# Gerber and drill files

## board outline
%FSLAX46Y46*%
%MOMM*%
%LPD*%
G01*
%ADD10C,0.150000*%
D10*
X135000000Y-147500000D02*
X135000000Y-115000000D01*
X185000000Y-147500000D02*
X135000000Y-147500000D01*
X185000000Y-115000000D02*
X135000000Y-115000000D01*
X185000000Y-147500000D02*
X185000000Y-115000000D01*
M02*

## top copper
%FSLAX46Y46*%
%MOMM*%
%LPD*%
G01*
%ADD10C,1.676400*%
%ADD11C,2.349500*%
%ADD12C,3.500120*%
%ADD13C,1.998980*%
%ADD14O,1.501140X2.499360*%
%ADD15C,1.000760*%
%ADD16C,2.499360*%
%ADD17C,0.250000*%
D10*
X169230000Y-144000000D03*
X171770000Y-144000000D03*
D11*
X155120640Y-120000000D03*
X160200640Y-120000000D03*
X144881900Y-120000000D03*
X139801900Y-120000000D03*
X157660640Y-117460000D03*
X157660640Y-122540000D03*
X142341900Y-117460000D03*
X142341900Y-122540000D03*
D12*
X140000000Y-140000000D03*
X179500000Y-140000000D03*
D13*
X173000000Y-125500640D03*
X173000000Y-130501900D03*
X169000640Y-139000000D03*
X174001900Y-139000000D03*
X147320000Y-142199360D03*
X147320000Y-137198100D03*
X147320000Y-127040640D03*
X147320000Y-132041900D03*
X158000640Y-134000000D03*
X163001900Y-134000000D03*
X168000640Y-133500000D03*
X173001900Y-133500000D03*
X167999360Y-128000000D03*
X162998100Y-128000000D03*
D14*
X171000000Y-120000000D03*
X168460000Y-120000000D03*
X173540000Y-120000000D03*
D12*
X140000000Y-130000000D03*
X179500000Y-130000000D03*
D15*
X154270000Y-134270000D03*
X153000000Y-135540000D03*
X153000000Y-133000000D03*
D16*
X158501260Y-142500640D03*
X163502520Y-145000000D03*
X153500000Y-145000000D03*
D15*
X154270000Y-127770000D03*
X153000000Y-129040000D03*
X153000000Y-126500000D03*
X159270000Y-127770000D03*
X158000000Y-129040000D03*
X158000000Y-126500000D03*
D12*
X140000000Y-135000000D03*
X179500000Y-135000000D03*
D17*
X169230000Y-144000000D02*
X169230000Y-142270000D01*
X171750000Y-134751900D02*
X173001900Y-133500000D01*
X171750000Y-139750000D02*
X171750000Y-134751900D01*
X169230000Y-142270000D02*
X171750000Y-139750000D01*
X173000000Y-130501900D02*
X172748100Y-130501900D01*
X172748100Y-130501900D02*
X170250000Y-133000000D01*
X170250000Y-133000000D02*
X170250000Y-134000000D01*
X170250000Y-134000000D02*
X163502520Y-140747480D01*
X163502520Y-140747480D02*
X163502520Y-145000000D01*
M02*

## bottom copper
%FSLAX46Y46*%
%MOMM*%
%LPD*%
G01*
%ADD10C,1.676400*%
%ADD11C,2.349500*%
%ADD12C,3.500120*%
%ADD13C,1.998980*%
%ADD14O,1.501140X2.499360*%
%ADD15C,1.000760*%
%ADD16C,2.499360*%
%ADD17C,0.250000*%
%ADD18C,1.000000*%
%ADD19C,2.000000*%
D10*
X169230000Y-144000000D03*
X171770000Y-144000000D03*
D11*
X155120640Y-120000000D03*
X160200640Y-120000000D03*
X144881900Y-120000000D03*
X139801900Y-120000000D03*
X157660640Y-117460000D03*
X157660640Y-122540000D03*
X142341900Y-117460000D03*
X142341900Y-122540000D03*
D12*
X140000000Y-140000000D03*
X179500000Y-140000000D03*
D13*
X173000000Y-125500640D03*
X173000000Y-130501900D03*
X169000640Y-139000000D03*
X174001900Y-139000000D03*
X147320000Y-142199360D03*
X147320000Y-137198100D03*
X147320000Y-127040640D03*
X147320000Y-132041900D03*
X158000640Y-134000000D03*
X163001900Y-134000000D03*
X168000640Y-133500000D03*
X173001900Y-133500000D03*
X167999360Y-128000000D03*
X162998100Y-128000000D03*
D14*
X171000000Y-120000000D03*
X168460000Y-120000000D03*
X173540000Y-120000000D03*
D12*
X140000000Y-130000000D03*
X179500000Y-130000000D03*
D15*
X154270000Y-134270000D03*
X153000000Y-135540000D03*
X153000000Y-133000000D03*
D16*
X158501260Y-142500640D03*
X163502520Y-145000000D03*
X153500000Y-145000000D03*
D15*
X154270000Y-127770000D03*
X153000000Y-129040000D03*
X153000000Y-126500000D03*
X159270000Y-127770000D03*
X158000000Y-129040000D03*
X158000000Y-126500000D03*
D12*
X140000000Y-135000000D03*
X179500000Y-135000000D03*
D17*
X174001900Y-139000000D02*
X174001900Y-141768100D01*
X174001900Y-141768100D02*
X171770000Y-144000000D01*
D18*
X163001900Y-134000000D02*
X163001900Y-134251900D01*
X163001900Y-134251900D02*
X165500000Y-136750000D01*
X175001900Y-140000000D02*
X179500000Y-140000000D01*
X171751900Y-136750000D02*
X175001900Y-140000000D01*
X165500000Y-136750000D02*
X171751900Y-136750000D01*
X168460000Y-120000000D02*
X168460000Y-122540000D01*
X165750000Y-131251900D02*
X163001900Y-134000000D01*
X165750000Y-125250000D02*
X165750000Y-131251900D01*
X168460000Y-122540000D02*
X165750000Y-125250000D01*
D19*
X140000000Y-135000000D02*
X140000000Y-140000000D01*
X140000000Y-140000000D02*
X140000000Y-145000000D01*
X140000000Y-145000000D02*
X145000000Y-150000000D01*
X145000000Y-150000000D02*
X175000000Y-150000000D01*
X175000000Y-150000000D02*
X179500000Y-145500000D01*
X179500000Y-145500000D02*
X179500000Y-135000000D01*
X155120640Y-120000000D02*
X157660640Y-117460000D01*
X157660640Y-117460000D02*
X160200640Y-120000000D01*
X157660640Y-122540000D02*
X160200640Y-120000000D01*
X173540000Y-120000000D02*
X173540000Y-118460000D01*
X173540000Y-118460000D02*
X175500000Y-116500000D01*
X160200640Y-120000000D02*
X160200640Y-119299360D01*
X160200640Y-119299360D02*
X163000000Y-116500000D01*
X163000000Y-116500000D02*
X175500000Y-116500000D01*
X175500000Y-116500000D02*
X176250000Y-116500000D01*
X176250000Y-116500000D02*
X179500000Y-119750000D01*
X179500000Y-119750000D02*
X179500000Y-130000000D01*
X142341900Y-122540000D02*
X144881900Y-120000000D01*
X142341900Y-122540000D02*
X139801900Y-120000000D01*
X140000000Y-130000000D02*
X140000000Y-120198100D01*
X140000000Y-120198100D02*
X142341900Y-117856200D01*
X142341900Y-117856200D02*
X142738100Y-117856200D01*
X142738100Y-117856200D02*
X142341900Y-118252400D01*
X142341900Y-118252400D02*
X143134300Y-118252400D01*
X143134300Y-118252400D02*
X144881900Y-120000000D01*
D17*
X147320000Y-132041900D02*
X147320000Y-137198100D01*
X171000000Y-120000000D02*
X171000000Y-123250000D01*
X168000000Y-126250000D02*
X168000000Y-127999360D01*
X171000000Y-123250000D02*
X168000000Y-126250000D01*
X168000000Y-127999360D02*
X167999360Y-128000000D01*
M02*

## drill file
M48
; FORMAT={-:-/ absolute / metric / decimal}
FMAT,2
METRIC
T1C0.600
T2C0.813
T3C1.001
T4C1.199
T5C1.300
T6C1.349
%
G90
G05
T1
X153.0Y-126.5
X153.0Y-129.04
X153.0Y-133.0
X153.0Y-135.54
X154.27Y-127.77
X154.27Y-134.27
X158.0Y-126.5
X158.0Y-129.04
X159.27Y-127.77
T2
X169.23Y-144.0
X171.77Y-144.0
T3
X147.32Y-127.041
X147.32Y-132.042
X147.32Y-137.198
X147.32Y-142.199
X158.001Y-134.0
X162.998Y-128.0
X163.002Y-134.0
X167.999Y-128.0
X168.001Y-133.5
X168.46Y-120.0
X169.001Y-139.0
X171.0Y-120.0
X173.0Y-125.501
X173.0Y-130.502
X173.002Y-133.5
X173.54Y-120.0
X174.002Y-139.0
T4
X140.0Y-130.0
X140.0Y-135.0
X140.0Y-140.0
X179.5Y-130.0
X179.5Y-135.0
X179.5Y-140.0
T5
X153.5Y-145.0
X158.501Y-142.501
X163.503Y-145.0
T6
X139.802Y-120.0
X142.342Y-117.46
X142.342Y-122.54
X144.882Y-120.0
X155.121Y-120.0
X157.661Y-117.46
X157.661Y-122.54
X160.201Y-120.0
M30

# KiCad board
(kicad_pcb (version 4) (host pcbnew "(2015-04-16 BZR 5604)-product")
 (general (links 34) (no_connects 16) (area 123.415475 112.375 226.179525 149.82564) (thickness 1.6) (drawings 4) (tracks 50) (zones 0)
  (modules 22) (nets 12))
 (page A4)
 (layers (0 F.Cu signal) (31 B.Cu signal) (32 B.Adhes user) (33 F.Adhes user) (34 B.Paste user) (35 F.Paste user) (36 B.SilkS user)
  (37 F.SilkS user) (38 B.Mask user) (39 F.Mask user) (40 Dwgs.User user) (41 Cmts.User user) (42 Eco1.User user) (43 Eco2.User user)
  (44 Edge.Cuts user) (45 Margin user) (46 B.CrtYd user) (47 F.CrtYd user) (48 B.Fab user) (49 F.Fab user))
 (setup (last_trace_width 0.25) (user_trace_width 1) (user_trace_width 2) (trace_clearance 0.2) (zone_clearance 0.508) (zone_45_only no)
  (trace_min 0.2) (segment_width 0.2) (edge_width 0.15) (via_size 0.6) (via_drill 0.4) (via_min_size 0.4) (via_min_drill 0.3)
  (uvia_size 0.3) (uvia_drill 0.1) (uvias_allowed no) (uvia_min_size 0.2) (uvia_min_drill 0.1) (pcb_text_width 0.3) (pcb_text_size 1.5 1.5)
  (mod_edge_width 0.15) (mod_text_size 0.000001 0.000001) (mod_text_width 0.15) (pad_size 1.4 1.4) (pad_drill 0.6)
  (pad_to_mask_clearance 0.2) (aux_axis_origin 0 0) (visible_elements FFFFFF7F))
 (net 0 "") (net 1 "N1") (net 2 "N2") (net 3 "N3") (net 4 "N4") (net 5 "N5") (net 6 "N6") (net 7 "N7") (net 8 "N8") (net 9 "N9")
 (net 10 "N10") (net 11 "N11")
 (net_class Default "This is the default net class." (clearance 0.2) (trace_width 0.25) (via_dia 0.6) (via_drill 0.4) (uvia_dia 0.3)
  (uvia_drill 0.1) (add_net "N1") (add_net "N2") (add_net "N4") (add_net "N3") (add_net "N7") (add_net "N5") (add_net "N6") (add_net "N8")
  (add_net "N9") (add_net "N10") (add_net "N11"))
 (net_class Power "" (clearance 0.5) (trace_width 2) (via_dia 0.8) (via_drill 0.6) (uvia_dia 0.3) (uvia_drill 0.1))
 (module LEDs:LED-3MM (layer F.Cu) (at 170.5 144)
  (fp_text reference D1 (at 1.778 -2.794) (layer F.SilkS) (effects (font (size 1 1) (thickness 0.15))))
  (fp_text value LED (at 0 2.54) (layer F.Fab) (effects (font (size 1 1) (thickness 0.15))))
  (pad 1 thru_hole circle (at -1.27 0) (size 1.6764 1.6764) (drill 0.8128) (layers *.Cu *.Mask F.SilkS) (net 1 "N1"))
  (pad 2 thru_hole circle (at 1.27 0) (size 1.6764 1.6764) (drill 0.8128) (layers *.Cu *.Mask F.SilkS) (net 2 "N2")))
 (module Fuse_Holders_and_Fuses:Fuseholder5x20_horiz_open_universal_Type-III (layer F.Cu) (at 150 120)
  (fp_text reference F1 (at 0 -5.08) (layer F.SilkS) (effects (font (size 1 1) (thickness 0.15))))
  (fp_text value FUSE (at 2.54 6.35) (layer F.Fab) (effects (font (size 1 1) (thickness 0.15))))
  (pad 2 thru_hole circle (at 5.12064 0) (size 2.3495 2.3495) (drill 1.34874) (layers *.Cu *.Mask F.SilkS) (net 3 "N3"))
  (pad 2 thru_hole circle (at 10.20064 0) (size 2.3495 2.3495) (drill 1.34874) (layers *.Cu *.Mask F.SilkS) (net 3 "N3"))
  (pad 1 thru_hole circle (at -5.1181 0) (size 2.3495 2.3495) (drill 1.34874) (layers *.Cu *.Mask F.SilkS) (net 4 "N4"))
  (pad 1 thru_hole circle (at -10.1981 0) (size 2.3495 2.3495) (drill 1.34874) (layers *.Cu *.Mask F.SilkS) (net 4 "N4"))
  (pad 2 thru_hole circle (at 7.66064 -2.54) (size 2.3495 2.3495) (drill 1.34874) (layers *.Cu *.Mask F.SilkS) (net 3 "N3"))
  (pad 2 thru_hole circle (at 7.66064 2.54) (size 2.3495 2.3495) (drill 1.34874) (layers *.Cu *.Mask F.SilkS) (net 3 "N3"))
  (pad 1 thru_hole circle (at -7.6581 -2.54) (size 2.3495 2.3495) (drill 1.34874) (layers *.Cu *.Mask F.SilkS) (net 4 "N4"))
  (pad 1 thru_hole circle (at -7.6581 2.54) (size 2.3495 2.3495) (drill 1.34874) (layers *.Cu *.Mask F.SilkS) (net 4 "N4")))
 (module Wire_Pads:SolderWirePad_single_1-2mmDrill (layer F.Cu) (at 140 140)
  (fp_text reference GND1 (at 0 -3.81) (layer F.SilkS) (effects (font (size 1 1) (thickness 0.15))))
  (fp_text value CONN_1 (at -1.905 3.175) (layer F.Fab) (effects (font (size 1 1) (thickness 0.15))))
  (pad 1 thru_hole circle (at 0 0) (size 3.50012 3.50012) (drill 1.19888) (layers *.Cu *.Mask F.SilkS) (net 2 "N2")))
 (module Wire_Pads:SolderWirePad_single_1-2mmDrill (layer F.Cu) (at 179.5 140)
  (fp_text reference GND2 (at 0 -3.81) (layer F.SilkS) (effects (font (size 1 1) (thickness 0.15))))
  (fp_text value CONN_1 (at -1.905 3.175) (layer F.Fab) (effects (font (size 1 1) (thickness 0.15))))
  (pad 1 thru_hole circle (at 0 0) (size 3.50012 3.50012) (drill 1.19888) (layers *.Cu *.Mask F.SilkS) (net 2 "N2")))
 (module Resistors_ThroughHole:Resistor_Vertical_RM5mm (layer F.Cu) (at 173 128 270)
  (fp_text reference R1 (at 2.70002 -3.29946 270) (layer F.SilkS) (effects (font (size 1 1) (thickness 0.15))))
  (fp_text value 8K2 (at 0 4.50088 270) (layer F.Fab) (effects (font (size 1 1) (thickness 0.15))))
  (pad 1 thru_hole circle (at -2.49936 0 270) (size 1.99898 1.99898) (drill 1.00076) (layers *.Cu *.SilkS *.Mask) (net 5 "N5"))
  (pad 2 thru_hole circle (at 2.5019 0 270) (size 1.99898 1.99898) (drill 1.00076) (layers *.Cu *.SilkS *.Mask) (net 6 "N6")))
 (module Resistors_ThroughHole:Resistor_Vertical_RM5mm (layer F.Cu) (at 171.5 139)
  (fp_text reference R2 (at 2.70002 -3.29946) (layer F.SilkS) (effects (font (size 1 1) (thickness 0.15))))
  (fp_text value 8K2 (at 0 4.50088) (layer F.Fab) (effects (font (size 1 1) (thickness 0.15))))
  (pad 1 thru_hole circle (at -2.49936 0) (size 1.99898 1.99898) (drill 1.00076) (layers *.Cu *.SilkS *.Mask) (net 5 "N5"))
  (pad 2 thru_hole circle (at 2.5019 0) (size 1.99898 1.99898) (drill 1.00076) (layers *.Cu *.SilkS *.Mask) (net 2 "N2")))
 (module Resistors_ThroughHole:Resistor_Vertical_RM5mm (layer F.Cu) (at 147.32 139.7 90)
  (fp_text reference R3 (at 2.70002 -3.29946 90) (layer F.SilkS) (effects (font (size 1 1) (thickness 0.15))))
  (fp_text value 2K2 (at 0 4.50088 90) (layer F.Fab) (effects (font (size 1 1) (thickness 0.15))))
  (pad 1 thru_hole circle (at -2.49936 0 90) (size 1.99898 1.99898) (drill 1.00076) (layers *.Cu *.SilkS *.Mask) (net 3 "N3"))
  (pad 2 thru_hole circle (at 2.5019 0 90) (size 1.99898 1.99898) (drill 1.00076) (layers *.Cu *.SilkS *.Mask) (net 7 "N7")))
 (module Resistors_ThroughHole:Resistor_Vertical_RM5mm (layer F.Cu) (at 147.32 129.54 270)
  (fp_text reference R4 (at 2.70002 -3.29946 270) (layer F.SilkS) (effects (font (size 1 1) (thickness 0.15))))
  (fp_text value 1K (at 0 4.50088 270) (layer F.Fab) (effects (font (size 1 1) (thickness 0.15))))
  (pad 1 thru_hole circle (at -2.49936 0 270) (size 1.99898 1.99898) (drill 1.00076) (layers *.Cu *.SilkS *.Mask) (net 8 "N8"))
  (pad 2 thru_hole circle (at 2.5019 0 270) (size 1.99898 1.99898) (drill 1.00076) (layers *.Cu *.SilkS *.Mask) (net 7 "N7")))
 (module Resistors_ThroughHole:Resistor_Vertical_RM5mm (layer F.Cu) (at 160.5 134)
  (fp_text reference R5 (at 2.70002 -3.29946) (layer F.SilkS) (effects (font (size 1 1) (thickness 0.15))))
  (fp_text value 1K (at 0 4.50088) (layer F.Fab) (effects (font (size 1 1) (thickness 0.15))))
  (pad 1 thru_hole circle (at -2.49936 0) (size 1.99898 1.99898) (drill 1.00076) (layers *.Cu *.SilkS *.Mask) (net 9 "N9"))
  (pad 2 thru_hole circle (at 2.5019 0) (size 1.99898 1.99898) (drill 1.00076) (layers *.Cu *.SilkS *.Mask) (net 2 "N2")))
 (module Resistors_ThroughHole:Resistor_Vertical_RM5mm (layer F.Cu) (at 170.5 133.5)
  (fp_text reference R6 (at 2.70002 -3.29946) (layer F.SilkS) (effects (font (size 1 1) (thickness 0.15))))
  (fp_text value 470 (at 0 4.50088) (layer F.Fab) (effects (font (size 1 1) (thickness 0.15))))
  (pad 1 thru_hole circle (at -2.49936 0) (size 1.99898 1.99898) (drill 1.00076) (layers *.Cu *.SilkS *.Mask) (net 9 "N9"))
  (pad 2 thru_hole circle (at 2.5019 0) (size 1.99898 1.99898) (drill 1.00076) (layers *.Cu *.SilkS *.Mask) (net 1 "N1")))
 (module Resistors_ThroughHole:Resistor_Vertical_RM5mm (layer F.Cu) (at 165.5 128 180)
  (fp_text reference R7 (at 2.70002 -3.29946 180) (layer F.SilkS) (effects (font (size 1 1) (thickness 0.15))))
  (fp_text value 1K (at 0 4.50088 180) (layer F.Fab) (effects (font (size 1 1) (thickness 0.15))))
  (pad 1 thru_hole circle (at -2.49936 0 180) (size 1.99898 1.99898) (drill 1.00076) (layers *.Cu *.SilkS *.Mask) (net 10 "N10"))
  (pad 2 thru_hole circle (at 2.5019 0 180) (size 1.99898 1.99898) (drill 1.00076) (layers *.Cu *.SilkS *.Mask) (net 9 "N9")))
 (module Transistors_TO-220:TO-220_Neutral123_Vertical (layer F.Cu) (at 171 120)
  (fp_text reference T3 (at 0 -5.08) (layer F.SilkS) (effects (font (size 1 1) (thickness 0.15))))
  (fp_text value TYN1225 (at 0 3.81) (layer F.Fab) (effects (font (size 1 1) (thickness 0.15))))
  (pad 2 thru_hole oval (at 0 0 90) (size 2.49936 1.50114) (drill 1.00076) (layers *.Cu *.Mask F.SilkS) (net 10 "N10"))
  (pad 1 thru_hole oval (at -2.54 0 90) (size 2.49936 1.50114) (drill 1.00076) (layers *.Cu *.Mask F.SilkS) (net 2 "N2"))
  (pad 3 thru_hole oval (at 2.54 0 90) (size 2.49936 1.50114) (drill 1.00076) (layers *.Cu *.Mask F.SilkS) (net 3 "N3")))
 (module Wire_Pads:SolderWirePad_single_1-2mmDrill (layer F.Cu) (at 140 130)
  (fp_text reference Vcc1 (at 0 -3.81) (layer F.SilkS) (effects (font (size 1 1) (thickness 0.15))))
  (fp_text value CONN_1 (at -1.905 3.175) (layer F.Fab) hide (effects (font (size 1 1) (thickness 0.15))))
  (pad 1 thru_hole circle (at 0 0) (size 3.50012 3.50012) (drill 1.19888) (layers *.Cu *.Mask F.SilkS) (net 4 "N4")))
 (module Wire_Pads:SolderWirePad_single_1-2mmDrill (layer F.Cu) (at 179.5 130)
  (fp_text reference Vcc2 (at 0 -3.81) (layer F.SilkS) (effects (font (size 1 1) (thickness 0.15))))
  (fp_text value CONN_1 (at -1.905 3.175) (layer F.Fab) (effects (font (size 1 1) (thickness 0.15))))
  (pad 1 thru_hole circle (at 0 0) (size 3.50012 3.50012) (drill 1.19888) (layers *.Cu *.Mask F.SilkS) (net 3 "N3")))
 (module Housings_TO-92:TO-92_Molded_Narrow (layer F.Cu) (at 153 133 270)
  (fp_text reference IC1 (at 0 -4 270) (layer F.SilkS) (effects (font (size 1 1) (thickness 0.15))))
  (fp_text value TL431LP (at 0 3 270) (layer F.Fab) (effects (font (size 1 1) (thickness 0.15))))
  (pad 2 thru_hole circle (at 1.27 -1.27) (size 1.00076 1.00076) (drill 0.6) (layers *.Cu *.Mask F.SilkS) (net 5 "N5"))
  (pad 3 thru_hole circle (at 2.54 0) (size 1.00076 1.00076) (drill 0.6) (layers *.Cu *.Mask F.SilkS) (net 2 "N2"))
  (pad 1 thru_hole circle (at 0 0) (size 1.00076 1.00076) (drill 0.6) (layers *.Cu *.Mask F.SilkS) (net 7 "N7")))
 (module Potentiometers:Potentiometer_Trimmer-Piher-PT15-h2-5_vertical (layer F.Cu) (at 153.5 145)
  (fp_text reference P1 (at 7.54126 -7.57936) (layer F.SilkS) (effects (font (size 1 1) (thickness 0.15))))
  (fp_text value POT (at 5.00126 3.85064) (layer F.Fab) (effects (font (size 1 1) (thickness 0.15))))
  (pad 2 thru_hole circle (at 5.00126 -2.49936) (size 2.49936 2.49936) (drill 1.30048) (layers *.Cu *.Mask F.SilkS) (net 3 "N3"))
  (pad 3 thru_hole circle (at 10.00252 0) (size 2.49936 2.49936) (drill 1.30048) (layers *.Cu *.Mask F.SilkS) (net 6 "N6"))
  (pad 1 thru_hole circle (at 0 0) (size 2.49936 2.49936) (drill 1.30048) (layers *.Cu *.Mask F.SilkS) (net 3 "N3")))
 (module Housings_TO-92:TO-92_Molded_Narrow (layer F.Cu) (at 153 126.5 270)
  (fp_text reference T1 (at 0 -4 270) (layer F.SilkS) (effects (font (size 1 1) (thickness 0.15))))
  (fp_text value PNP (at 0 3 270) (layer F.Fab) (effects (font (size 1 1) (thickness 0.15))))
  (pad 2 thru_hole circle (at 1.27 -1.27) (size 1.00076 1.00076) (drill 0.6) (layers *.Cu *.Mask F.SilkS) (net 8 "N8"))
  (pad 3 thru_hole circle (at 2.54 0) (size 1.00076 1.00076) (drill 0.6) (layers *.Cu *.Mask F.SilkS) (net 2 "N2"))
  (pad 1 thru_hole circle (at 0 0) (size 1.00076 1.00076) (drill 0.6) (layers *.Cu *.Mask F.SilkS) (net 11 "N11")))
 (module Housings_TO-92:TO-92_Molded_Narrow (layer F.Cu) (at 158 126.5 270)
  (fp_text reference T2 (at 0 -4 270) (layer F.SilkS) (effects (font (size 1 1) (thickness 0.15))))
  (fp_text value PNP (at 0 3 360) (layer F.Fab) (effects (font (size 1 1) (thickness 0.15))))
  (pad 2 thru_hole circle (at 1.27 -1.27) (size 1.00076 1.00076) (drill 0.6) (layers *.Cu *.Mask F.SilkS) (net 11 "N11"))
  (pad 3 thru_hole circle (at 2.54 0) (size 1.00076 1.00076) (drill 0.6) (layers *.Cu *.Mask F.SilkS) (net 9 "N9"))
  (pad 1 thru_hole circle (at 0 0) (size 1.00076 1.00076) (drill 0.6) (layers *.Cu *.Mask F.SilkS) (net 3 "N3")))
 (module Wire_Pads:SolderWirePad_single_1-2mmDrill (layer F.Cu) (at 215 127.5)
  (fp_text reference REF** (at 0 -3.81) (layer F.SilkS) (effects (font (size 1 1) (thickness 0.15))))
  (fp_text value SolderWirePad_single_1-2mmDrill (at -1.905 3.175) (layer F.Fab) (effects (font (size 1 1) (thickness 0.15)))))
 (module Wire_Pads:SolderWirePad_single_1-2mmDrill (layer F.Cu) (at 140 127.5)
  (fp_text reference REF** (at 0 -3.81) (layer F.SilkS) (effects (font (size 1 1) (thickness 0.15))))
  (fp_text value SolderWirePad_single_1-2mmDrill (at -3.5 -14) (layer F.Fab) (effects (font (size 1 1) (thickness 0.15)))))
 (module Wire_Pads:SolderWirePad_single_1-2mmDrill (layer F.Cu) (at 140 135)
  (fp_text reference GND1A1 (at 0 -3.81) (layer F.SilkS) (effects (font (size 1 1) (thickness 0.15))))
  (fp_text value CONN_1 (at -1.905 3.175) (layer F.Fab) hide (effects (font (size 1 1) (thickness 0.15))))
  (pad 1 thru_hole circle (at 0 0) (size 3.50012 3.50012) (drill 1.19888) (layers *.Cu *.Mask F.SilkS) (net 2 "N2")))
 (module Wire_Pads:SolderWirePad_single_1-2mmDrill (layer F.Cu) (at 179.5 135)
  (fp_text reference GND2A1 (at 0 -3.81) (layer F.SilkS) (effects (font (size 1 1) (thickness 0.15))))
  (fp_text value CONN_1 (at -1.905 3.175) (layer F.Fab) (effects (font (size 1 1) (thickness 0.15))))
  (pad 1 thru_hole circle (at 0 0) (size 3.50012 3.50012) (drill 1.19888) (layers *.Cu *.Mask F.SilkS) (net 2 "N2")))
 (gr_line (start 135 147.5) (end 135 115) (angle 90) (layer Edge.Cuts) (width 0.15))
 (gr_line (start 185 147.5) (end 135 147.5) (angle 90) (layer Edge.Cuts) (width 0.15))
 (gr_line (start 185 115) (end 135 115) (angle 90) (layer Edge.Cuts) (width 0.15))
 (gr_line (start 185 147.5) (end 185 115) (angle 90) (layer Edge.Cuts) (width 0.15))
 (segment (start 169.23 144) (end 169.23 142.27) (width 0.25) (layer F.Cu) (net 1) (status 400000))
 (segment (start 171.75 134.7519) (end 173.0019 133.5) (width 0.25) (layer F.Cu) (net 1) (status 800000))
 (segment (start 171.75 139.75) (end 171.75 134.7519) (width 0.25) (layer F.Cu) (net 1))
 (segment (start 169.23 142.27) (end 171.75 139.75) (width 0.25) (layer F.Cu) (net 1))
 (segment (start 174.0019 139) (end 174.0019 141.7681) (width 0.25) (layer B.Cu) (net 2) (status 400000))
 (segment (start 174.0019 141.7681) (end 171.77 144) (width 0.25) (layer B.Cu) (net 2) (status 800000))
 (segment (start 163.0019 134) (end 163.0019 134.2519) (width 1) (layer B.Cu) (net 2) (status C00000))
 (segment (start 163.0019 134.2519) (end 165.5 136.75) (width 1) (layer B.Cu) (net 2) (status 400000))
 (segment (start 175.0019 140) (end 179.5 140) (width 1) (layer B.Cu) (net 2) (status 800000))
 (segment (start 171.7519 136.75) (end 175.0019 140) (width 1) (layer B.Cu) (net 2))
 (segment (start 165.5 136.75) (end 171.7519 136.75) (width 1) (layer B.Cu) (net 2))
 (segment (start 168.46 120) (end 168.46 122.54) (width 1) (layer B.Cu) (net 2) (status 400000))
 (segment (start 165.75 131.2519) (end 163.0019 134) (width 1) (layer B.Cu) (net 2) (status 800000))
 (segment (start 165.75 125.25) (end 165.75 131.2519) (width 1) (layer B.Cu) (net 2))
 (segment (start 168.46 122.54) (end 165.75 125.25) (width 1) (layer B.Cu) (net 2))
 (segment (start 140 135) (end 140 140) (width 2) (layer B.Cu) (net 2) (status C00000))
 (segment (start 140 140) (end 140 145) (width 2) (layer B.Cu) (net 2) (status 400000))
 (segment (start 140 145) (end 145 150) (width 2) (layer B.Cu) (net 2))
 (segment (start 145 150) (end 175 150) (width 2) (layer B.Cu) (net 2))
 (segment (start 175 150) (end 179.5 145.5) (width 2) (layer B.Cu) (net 2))
 (segment (start 179.5 145.5) (end 179.5 135) (width 2) (layer B.Cu) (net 2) (status 800000))
 (segment (start 155.12064 120) (end 157.66064 117.46) (width 2) (layer B.Cu) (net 3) (status C00000))
 (segment (start 157.66064 117.46) (end 160.20064 120) (width 2) (layer B.Cu) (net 3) (status C00000))
 (segment (start 157.66064 122.54) (end 160.20064 120) (width 2) (layer B.Cu) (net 3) (status C00000))
 (segment (start 173.54 120) (end 173.54 118.46) (width 2) (layer B.Cu) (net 3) (status 400000))
 (segment (start 173.54 118.46) (end 175.5 116.5) (width 2) (layer B.Cu) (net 3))
 (segment (start 160.20064 120) (end 160.20064 119.29936) (width 2) (layer B.Cu) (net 3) (status C00000))
 (segment (start 160.20064 119.29936) (end 163 116.5) (width 2) (layer B.Cu) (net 3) (status 400000))
 (segment (start 163 116.5) (end 175.5 116.5) (width 2) (layer B.Cu) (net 3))
 (segment (start 175.5 116.5) (end 176.25 116.5) (width 2) (layer B.Cu) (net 3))
 (segment (start 176.25 116.5) (end 179.5 119.75) (width 2) (layer B.Cu) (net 3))
 (segment (start 179.5 119.75) (end 179.5 130) (width 2) (layer B.Cu) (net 3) (status 800000))
 (segment (start 142.3419 122.54) (end 144.8819 120) (width 2) (layer B.Cu) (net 4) (status C00000))
 (segment (start 142.3419 122.54) (end 139.8019 120) (width 2) (layer B.Cu) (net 4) (status C00000))
 (segment (start 140 130) (end 140 120.1981) (width 2) (layer B.Cu) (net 4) (status C00000))
 (segment (start 140 120.1981) (end 142.3419 117.8562) (width 2) (layer B.Cu) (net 4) (status C00000))
 (segment (start 142.3419 117.8562) (end 142.7381 117.8562) (width 2) (layer B.Cu) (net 4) (status C00000))
 (segment (start 142.7381 117.8562) (end 142.3419 118.2524) (width 2) (layer B.Cu) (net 4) (status C00000))
 (segment (start 142.3419 118.2524) (end 143.1343 118.2524) (width 2) (layer B.Cu) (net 4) (status C00000))
 (segment (start 143.1343 118.2524) (end 144.8819 120) (width 2) (layer B.Cu) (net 4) (status C00000))
 (segment (start 147.32 132.0419) (end 147.32 137.1981) (width 0.25) (layer B.Cu) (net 7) (status C00000))
 (segment (start 173 130.5019) (end 172.7481 130.5019) (width 0.25) (layer F.Cu) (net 6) (status C00000))
 (segment (start 172.7481 130.5019) (end 170.25 133) (width 0.25) (layer F.Cu) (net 6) (status 400000))
 (segment (start 170.25 133) (end 170.25 134) (width 0.25) (layer F.Cu) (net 6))
 (segment (start 170.25 134) (end 163.50252 140.74748) (width 0.25) (layer F.Cu) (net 6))
 (segment (start 163.50252 140.74748) (end 163.50252 145) (width 0.25) (layer F.Cu) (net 6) (status 800000))
 (segment (start 171 120) (end 171 123.25) (width 0.25) (layer B.Cu) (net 10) (status 400000))
 (segment (start 168 126.25) (end 168 127.99936) (width 0.25) (layer B.Cu) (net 10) (status 800000))
 (segment (start 171 123.25) (end 168 126.25) (width 0.25) (layer B.Cu) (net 10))
 (segment (start 168 127.99936) (end 167.99936 128) (width 0.25) (layer B.Cu) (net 10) (status C00000)))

